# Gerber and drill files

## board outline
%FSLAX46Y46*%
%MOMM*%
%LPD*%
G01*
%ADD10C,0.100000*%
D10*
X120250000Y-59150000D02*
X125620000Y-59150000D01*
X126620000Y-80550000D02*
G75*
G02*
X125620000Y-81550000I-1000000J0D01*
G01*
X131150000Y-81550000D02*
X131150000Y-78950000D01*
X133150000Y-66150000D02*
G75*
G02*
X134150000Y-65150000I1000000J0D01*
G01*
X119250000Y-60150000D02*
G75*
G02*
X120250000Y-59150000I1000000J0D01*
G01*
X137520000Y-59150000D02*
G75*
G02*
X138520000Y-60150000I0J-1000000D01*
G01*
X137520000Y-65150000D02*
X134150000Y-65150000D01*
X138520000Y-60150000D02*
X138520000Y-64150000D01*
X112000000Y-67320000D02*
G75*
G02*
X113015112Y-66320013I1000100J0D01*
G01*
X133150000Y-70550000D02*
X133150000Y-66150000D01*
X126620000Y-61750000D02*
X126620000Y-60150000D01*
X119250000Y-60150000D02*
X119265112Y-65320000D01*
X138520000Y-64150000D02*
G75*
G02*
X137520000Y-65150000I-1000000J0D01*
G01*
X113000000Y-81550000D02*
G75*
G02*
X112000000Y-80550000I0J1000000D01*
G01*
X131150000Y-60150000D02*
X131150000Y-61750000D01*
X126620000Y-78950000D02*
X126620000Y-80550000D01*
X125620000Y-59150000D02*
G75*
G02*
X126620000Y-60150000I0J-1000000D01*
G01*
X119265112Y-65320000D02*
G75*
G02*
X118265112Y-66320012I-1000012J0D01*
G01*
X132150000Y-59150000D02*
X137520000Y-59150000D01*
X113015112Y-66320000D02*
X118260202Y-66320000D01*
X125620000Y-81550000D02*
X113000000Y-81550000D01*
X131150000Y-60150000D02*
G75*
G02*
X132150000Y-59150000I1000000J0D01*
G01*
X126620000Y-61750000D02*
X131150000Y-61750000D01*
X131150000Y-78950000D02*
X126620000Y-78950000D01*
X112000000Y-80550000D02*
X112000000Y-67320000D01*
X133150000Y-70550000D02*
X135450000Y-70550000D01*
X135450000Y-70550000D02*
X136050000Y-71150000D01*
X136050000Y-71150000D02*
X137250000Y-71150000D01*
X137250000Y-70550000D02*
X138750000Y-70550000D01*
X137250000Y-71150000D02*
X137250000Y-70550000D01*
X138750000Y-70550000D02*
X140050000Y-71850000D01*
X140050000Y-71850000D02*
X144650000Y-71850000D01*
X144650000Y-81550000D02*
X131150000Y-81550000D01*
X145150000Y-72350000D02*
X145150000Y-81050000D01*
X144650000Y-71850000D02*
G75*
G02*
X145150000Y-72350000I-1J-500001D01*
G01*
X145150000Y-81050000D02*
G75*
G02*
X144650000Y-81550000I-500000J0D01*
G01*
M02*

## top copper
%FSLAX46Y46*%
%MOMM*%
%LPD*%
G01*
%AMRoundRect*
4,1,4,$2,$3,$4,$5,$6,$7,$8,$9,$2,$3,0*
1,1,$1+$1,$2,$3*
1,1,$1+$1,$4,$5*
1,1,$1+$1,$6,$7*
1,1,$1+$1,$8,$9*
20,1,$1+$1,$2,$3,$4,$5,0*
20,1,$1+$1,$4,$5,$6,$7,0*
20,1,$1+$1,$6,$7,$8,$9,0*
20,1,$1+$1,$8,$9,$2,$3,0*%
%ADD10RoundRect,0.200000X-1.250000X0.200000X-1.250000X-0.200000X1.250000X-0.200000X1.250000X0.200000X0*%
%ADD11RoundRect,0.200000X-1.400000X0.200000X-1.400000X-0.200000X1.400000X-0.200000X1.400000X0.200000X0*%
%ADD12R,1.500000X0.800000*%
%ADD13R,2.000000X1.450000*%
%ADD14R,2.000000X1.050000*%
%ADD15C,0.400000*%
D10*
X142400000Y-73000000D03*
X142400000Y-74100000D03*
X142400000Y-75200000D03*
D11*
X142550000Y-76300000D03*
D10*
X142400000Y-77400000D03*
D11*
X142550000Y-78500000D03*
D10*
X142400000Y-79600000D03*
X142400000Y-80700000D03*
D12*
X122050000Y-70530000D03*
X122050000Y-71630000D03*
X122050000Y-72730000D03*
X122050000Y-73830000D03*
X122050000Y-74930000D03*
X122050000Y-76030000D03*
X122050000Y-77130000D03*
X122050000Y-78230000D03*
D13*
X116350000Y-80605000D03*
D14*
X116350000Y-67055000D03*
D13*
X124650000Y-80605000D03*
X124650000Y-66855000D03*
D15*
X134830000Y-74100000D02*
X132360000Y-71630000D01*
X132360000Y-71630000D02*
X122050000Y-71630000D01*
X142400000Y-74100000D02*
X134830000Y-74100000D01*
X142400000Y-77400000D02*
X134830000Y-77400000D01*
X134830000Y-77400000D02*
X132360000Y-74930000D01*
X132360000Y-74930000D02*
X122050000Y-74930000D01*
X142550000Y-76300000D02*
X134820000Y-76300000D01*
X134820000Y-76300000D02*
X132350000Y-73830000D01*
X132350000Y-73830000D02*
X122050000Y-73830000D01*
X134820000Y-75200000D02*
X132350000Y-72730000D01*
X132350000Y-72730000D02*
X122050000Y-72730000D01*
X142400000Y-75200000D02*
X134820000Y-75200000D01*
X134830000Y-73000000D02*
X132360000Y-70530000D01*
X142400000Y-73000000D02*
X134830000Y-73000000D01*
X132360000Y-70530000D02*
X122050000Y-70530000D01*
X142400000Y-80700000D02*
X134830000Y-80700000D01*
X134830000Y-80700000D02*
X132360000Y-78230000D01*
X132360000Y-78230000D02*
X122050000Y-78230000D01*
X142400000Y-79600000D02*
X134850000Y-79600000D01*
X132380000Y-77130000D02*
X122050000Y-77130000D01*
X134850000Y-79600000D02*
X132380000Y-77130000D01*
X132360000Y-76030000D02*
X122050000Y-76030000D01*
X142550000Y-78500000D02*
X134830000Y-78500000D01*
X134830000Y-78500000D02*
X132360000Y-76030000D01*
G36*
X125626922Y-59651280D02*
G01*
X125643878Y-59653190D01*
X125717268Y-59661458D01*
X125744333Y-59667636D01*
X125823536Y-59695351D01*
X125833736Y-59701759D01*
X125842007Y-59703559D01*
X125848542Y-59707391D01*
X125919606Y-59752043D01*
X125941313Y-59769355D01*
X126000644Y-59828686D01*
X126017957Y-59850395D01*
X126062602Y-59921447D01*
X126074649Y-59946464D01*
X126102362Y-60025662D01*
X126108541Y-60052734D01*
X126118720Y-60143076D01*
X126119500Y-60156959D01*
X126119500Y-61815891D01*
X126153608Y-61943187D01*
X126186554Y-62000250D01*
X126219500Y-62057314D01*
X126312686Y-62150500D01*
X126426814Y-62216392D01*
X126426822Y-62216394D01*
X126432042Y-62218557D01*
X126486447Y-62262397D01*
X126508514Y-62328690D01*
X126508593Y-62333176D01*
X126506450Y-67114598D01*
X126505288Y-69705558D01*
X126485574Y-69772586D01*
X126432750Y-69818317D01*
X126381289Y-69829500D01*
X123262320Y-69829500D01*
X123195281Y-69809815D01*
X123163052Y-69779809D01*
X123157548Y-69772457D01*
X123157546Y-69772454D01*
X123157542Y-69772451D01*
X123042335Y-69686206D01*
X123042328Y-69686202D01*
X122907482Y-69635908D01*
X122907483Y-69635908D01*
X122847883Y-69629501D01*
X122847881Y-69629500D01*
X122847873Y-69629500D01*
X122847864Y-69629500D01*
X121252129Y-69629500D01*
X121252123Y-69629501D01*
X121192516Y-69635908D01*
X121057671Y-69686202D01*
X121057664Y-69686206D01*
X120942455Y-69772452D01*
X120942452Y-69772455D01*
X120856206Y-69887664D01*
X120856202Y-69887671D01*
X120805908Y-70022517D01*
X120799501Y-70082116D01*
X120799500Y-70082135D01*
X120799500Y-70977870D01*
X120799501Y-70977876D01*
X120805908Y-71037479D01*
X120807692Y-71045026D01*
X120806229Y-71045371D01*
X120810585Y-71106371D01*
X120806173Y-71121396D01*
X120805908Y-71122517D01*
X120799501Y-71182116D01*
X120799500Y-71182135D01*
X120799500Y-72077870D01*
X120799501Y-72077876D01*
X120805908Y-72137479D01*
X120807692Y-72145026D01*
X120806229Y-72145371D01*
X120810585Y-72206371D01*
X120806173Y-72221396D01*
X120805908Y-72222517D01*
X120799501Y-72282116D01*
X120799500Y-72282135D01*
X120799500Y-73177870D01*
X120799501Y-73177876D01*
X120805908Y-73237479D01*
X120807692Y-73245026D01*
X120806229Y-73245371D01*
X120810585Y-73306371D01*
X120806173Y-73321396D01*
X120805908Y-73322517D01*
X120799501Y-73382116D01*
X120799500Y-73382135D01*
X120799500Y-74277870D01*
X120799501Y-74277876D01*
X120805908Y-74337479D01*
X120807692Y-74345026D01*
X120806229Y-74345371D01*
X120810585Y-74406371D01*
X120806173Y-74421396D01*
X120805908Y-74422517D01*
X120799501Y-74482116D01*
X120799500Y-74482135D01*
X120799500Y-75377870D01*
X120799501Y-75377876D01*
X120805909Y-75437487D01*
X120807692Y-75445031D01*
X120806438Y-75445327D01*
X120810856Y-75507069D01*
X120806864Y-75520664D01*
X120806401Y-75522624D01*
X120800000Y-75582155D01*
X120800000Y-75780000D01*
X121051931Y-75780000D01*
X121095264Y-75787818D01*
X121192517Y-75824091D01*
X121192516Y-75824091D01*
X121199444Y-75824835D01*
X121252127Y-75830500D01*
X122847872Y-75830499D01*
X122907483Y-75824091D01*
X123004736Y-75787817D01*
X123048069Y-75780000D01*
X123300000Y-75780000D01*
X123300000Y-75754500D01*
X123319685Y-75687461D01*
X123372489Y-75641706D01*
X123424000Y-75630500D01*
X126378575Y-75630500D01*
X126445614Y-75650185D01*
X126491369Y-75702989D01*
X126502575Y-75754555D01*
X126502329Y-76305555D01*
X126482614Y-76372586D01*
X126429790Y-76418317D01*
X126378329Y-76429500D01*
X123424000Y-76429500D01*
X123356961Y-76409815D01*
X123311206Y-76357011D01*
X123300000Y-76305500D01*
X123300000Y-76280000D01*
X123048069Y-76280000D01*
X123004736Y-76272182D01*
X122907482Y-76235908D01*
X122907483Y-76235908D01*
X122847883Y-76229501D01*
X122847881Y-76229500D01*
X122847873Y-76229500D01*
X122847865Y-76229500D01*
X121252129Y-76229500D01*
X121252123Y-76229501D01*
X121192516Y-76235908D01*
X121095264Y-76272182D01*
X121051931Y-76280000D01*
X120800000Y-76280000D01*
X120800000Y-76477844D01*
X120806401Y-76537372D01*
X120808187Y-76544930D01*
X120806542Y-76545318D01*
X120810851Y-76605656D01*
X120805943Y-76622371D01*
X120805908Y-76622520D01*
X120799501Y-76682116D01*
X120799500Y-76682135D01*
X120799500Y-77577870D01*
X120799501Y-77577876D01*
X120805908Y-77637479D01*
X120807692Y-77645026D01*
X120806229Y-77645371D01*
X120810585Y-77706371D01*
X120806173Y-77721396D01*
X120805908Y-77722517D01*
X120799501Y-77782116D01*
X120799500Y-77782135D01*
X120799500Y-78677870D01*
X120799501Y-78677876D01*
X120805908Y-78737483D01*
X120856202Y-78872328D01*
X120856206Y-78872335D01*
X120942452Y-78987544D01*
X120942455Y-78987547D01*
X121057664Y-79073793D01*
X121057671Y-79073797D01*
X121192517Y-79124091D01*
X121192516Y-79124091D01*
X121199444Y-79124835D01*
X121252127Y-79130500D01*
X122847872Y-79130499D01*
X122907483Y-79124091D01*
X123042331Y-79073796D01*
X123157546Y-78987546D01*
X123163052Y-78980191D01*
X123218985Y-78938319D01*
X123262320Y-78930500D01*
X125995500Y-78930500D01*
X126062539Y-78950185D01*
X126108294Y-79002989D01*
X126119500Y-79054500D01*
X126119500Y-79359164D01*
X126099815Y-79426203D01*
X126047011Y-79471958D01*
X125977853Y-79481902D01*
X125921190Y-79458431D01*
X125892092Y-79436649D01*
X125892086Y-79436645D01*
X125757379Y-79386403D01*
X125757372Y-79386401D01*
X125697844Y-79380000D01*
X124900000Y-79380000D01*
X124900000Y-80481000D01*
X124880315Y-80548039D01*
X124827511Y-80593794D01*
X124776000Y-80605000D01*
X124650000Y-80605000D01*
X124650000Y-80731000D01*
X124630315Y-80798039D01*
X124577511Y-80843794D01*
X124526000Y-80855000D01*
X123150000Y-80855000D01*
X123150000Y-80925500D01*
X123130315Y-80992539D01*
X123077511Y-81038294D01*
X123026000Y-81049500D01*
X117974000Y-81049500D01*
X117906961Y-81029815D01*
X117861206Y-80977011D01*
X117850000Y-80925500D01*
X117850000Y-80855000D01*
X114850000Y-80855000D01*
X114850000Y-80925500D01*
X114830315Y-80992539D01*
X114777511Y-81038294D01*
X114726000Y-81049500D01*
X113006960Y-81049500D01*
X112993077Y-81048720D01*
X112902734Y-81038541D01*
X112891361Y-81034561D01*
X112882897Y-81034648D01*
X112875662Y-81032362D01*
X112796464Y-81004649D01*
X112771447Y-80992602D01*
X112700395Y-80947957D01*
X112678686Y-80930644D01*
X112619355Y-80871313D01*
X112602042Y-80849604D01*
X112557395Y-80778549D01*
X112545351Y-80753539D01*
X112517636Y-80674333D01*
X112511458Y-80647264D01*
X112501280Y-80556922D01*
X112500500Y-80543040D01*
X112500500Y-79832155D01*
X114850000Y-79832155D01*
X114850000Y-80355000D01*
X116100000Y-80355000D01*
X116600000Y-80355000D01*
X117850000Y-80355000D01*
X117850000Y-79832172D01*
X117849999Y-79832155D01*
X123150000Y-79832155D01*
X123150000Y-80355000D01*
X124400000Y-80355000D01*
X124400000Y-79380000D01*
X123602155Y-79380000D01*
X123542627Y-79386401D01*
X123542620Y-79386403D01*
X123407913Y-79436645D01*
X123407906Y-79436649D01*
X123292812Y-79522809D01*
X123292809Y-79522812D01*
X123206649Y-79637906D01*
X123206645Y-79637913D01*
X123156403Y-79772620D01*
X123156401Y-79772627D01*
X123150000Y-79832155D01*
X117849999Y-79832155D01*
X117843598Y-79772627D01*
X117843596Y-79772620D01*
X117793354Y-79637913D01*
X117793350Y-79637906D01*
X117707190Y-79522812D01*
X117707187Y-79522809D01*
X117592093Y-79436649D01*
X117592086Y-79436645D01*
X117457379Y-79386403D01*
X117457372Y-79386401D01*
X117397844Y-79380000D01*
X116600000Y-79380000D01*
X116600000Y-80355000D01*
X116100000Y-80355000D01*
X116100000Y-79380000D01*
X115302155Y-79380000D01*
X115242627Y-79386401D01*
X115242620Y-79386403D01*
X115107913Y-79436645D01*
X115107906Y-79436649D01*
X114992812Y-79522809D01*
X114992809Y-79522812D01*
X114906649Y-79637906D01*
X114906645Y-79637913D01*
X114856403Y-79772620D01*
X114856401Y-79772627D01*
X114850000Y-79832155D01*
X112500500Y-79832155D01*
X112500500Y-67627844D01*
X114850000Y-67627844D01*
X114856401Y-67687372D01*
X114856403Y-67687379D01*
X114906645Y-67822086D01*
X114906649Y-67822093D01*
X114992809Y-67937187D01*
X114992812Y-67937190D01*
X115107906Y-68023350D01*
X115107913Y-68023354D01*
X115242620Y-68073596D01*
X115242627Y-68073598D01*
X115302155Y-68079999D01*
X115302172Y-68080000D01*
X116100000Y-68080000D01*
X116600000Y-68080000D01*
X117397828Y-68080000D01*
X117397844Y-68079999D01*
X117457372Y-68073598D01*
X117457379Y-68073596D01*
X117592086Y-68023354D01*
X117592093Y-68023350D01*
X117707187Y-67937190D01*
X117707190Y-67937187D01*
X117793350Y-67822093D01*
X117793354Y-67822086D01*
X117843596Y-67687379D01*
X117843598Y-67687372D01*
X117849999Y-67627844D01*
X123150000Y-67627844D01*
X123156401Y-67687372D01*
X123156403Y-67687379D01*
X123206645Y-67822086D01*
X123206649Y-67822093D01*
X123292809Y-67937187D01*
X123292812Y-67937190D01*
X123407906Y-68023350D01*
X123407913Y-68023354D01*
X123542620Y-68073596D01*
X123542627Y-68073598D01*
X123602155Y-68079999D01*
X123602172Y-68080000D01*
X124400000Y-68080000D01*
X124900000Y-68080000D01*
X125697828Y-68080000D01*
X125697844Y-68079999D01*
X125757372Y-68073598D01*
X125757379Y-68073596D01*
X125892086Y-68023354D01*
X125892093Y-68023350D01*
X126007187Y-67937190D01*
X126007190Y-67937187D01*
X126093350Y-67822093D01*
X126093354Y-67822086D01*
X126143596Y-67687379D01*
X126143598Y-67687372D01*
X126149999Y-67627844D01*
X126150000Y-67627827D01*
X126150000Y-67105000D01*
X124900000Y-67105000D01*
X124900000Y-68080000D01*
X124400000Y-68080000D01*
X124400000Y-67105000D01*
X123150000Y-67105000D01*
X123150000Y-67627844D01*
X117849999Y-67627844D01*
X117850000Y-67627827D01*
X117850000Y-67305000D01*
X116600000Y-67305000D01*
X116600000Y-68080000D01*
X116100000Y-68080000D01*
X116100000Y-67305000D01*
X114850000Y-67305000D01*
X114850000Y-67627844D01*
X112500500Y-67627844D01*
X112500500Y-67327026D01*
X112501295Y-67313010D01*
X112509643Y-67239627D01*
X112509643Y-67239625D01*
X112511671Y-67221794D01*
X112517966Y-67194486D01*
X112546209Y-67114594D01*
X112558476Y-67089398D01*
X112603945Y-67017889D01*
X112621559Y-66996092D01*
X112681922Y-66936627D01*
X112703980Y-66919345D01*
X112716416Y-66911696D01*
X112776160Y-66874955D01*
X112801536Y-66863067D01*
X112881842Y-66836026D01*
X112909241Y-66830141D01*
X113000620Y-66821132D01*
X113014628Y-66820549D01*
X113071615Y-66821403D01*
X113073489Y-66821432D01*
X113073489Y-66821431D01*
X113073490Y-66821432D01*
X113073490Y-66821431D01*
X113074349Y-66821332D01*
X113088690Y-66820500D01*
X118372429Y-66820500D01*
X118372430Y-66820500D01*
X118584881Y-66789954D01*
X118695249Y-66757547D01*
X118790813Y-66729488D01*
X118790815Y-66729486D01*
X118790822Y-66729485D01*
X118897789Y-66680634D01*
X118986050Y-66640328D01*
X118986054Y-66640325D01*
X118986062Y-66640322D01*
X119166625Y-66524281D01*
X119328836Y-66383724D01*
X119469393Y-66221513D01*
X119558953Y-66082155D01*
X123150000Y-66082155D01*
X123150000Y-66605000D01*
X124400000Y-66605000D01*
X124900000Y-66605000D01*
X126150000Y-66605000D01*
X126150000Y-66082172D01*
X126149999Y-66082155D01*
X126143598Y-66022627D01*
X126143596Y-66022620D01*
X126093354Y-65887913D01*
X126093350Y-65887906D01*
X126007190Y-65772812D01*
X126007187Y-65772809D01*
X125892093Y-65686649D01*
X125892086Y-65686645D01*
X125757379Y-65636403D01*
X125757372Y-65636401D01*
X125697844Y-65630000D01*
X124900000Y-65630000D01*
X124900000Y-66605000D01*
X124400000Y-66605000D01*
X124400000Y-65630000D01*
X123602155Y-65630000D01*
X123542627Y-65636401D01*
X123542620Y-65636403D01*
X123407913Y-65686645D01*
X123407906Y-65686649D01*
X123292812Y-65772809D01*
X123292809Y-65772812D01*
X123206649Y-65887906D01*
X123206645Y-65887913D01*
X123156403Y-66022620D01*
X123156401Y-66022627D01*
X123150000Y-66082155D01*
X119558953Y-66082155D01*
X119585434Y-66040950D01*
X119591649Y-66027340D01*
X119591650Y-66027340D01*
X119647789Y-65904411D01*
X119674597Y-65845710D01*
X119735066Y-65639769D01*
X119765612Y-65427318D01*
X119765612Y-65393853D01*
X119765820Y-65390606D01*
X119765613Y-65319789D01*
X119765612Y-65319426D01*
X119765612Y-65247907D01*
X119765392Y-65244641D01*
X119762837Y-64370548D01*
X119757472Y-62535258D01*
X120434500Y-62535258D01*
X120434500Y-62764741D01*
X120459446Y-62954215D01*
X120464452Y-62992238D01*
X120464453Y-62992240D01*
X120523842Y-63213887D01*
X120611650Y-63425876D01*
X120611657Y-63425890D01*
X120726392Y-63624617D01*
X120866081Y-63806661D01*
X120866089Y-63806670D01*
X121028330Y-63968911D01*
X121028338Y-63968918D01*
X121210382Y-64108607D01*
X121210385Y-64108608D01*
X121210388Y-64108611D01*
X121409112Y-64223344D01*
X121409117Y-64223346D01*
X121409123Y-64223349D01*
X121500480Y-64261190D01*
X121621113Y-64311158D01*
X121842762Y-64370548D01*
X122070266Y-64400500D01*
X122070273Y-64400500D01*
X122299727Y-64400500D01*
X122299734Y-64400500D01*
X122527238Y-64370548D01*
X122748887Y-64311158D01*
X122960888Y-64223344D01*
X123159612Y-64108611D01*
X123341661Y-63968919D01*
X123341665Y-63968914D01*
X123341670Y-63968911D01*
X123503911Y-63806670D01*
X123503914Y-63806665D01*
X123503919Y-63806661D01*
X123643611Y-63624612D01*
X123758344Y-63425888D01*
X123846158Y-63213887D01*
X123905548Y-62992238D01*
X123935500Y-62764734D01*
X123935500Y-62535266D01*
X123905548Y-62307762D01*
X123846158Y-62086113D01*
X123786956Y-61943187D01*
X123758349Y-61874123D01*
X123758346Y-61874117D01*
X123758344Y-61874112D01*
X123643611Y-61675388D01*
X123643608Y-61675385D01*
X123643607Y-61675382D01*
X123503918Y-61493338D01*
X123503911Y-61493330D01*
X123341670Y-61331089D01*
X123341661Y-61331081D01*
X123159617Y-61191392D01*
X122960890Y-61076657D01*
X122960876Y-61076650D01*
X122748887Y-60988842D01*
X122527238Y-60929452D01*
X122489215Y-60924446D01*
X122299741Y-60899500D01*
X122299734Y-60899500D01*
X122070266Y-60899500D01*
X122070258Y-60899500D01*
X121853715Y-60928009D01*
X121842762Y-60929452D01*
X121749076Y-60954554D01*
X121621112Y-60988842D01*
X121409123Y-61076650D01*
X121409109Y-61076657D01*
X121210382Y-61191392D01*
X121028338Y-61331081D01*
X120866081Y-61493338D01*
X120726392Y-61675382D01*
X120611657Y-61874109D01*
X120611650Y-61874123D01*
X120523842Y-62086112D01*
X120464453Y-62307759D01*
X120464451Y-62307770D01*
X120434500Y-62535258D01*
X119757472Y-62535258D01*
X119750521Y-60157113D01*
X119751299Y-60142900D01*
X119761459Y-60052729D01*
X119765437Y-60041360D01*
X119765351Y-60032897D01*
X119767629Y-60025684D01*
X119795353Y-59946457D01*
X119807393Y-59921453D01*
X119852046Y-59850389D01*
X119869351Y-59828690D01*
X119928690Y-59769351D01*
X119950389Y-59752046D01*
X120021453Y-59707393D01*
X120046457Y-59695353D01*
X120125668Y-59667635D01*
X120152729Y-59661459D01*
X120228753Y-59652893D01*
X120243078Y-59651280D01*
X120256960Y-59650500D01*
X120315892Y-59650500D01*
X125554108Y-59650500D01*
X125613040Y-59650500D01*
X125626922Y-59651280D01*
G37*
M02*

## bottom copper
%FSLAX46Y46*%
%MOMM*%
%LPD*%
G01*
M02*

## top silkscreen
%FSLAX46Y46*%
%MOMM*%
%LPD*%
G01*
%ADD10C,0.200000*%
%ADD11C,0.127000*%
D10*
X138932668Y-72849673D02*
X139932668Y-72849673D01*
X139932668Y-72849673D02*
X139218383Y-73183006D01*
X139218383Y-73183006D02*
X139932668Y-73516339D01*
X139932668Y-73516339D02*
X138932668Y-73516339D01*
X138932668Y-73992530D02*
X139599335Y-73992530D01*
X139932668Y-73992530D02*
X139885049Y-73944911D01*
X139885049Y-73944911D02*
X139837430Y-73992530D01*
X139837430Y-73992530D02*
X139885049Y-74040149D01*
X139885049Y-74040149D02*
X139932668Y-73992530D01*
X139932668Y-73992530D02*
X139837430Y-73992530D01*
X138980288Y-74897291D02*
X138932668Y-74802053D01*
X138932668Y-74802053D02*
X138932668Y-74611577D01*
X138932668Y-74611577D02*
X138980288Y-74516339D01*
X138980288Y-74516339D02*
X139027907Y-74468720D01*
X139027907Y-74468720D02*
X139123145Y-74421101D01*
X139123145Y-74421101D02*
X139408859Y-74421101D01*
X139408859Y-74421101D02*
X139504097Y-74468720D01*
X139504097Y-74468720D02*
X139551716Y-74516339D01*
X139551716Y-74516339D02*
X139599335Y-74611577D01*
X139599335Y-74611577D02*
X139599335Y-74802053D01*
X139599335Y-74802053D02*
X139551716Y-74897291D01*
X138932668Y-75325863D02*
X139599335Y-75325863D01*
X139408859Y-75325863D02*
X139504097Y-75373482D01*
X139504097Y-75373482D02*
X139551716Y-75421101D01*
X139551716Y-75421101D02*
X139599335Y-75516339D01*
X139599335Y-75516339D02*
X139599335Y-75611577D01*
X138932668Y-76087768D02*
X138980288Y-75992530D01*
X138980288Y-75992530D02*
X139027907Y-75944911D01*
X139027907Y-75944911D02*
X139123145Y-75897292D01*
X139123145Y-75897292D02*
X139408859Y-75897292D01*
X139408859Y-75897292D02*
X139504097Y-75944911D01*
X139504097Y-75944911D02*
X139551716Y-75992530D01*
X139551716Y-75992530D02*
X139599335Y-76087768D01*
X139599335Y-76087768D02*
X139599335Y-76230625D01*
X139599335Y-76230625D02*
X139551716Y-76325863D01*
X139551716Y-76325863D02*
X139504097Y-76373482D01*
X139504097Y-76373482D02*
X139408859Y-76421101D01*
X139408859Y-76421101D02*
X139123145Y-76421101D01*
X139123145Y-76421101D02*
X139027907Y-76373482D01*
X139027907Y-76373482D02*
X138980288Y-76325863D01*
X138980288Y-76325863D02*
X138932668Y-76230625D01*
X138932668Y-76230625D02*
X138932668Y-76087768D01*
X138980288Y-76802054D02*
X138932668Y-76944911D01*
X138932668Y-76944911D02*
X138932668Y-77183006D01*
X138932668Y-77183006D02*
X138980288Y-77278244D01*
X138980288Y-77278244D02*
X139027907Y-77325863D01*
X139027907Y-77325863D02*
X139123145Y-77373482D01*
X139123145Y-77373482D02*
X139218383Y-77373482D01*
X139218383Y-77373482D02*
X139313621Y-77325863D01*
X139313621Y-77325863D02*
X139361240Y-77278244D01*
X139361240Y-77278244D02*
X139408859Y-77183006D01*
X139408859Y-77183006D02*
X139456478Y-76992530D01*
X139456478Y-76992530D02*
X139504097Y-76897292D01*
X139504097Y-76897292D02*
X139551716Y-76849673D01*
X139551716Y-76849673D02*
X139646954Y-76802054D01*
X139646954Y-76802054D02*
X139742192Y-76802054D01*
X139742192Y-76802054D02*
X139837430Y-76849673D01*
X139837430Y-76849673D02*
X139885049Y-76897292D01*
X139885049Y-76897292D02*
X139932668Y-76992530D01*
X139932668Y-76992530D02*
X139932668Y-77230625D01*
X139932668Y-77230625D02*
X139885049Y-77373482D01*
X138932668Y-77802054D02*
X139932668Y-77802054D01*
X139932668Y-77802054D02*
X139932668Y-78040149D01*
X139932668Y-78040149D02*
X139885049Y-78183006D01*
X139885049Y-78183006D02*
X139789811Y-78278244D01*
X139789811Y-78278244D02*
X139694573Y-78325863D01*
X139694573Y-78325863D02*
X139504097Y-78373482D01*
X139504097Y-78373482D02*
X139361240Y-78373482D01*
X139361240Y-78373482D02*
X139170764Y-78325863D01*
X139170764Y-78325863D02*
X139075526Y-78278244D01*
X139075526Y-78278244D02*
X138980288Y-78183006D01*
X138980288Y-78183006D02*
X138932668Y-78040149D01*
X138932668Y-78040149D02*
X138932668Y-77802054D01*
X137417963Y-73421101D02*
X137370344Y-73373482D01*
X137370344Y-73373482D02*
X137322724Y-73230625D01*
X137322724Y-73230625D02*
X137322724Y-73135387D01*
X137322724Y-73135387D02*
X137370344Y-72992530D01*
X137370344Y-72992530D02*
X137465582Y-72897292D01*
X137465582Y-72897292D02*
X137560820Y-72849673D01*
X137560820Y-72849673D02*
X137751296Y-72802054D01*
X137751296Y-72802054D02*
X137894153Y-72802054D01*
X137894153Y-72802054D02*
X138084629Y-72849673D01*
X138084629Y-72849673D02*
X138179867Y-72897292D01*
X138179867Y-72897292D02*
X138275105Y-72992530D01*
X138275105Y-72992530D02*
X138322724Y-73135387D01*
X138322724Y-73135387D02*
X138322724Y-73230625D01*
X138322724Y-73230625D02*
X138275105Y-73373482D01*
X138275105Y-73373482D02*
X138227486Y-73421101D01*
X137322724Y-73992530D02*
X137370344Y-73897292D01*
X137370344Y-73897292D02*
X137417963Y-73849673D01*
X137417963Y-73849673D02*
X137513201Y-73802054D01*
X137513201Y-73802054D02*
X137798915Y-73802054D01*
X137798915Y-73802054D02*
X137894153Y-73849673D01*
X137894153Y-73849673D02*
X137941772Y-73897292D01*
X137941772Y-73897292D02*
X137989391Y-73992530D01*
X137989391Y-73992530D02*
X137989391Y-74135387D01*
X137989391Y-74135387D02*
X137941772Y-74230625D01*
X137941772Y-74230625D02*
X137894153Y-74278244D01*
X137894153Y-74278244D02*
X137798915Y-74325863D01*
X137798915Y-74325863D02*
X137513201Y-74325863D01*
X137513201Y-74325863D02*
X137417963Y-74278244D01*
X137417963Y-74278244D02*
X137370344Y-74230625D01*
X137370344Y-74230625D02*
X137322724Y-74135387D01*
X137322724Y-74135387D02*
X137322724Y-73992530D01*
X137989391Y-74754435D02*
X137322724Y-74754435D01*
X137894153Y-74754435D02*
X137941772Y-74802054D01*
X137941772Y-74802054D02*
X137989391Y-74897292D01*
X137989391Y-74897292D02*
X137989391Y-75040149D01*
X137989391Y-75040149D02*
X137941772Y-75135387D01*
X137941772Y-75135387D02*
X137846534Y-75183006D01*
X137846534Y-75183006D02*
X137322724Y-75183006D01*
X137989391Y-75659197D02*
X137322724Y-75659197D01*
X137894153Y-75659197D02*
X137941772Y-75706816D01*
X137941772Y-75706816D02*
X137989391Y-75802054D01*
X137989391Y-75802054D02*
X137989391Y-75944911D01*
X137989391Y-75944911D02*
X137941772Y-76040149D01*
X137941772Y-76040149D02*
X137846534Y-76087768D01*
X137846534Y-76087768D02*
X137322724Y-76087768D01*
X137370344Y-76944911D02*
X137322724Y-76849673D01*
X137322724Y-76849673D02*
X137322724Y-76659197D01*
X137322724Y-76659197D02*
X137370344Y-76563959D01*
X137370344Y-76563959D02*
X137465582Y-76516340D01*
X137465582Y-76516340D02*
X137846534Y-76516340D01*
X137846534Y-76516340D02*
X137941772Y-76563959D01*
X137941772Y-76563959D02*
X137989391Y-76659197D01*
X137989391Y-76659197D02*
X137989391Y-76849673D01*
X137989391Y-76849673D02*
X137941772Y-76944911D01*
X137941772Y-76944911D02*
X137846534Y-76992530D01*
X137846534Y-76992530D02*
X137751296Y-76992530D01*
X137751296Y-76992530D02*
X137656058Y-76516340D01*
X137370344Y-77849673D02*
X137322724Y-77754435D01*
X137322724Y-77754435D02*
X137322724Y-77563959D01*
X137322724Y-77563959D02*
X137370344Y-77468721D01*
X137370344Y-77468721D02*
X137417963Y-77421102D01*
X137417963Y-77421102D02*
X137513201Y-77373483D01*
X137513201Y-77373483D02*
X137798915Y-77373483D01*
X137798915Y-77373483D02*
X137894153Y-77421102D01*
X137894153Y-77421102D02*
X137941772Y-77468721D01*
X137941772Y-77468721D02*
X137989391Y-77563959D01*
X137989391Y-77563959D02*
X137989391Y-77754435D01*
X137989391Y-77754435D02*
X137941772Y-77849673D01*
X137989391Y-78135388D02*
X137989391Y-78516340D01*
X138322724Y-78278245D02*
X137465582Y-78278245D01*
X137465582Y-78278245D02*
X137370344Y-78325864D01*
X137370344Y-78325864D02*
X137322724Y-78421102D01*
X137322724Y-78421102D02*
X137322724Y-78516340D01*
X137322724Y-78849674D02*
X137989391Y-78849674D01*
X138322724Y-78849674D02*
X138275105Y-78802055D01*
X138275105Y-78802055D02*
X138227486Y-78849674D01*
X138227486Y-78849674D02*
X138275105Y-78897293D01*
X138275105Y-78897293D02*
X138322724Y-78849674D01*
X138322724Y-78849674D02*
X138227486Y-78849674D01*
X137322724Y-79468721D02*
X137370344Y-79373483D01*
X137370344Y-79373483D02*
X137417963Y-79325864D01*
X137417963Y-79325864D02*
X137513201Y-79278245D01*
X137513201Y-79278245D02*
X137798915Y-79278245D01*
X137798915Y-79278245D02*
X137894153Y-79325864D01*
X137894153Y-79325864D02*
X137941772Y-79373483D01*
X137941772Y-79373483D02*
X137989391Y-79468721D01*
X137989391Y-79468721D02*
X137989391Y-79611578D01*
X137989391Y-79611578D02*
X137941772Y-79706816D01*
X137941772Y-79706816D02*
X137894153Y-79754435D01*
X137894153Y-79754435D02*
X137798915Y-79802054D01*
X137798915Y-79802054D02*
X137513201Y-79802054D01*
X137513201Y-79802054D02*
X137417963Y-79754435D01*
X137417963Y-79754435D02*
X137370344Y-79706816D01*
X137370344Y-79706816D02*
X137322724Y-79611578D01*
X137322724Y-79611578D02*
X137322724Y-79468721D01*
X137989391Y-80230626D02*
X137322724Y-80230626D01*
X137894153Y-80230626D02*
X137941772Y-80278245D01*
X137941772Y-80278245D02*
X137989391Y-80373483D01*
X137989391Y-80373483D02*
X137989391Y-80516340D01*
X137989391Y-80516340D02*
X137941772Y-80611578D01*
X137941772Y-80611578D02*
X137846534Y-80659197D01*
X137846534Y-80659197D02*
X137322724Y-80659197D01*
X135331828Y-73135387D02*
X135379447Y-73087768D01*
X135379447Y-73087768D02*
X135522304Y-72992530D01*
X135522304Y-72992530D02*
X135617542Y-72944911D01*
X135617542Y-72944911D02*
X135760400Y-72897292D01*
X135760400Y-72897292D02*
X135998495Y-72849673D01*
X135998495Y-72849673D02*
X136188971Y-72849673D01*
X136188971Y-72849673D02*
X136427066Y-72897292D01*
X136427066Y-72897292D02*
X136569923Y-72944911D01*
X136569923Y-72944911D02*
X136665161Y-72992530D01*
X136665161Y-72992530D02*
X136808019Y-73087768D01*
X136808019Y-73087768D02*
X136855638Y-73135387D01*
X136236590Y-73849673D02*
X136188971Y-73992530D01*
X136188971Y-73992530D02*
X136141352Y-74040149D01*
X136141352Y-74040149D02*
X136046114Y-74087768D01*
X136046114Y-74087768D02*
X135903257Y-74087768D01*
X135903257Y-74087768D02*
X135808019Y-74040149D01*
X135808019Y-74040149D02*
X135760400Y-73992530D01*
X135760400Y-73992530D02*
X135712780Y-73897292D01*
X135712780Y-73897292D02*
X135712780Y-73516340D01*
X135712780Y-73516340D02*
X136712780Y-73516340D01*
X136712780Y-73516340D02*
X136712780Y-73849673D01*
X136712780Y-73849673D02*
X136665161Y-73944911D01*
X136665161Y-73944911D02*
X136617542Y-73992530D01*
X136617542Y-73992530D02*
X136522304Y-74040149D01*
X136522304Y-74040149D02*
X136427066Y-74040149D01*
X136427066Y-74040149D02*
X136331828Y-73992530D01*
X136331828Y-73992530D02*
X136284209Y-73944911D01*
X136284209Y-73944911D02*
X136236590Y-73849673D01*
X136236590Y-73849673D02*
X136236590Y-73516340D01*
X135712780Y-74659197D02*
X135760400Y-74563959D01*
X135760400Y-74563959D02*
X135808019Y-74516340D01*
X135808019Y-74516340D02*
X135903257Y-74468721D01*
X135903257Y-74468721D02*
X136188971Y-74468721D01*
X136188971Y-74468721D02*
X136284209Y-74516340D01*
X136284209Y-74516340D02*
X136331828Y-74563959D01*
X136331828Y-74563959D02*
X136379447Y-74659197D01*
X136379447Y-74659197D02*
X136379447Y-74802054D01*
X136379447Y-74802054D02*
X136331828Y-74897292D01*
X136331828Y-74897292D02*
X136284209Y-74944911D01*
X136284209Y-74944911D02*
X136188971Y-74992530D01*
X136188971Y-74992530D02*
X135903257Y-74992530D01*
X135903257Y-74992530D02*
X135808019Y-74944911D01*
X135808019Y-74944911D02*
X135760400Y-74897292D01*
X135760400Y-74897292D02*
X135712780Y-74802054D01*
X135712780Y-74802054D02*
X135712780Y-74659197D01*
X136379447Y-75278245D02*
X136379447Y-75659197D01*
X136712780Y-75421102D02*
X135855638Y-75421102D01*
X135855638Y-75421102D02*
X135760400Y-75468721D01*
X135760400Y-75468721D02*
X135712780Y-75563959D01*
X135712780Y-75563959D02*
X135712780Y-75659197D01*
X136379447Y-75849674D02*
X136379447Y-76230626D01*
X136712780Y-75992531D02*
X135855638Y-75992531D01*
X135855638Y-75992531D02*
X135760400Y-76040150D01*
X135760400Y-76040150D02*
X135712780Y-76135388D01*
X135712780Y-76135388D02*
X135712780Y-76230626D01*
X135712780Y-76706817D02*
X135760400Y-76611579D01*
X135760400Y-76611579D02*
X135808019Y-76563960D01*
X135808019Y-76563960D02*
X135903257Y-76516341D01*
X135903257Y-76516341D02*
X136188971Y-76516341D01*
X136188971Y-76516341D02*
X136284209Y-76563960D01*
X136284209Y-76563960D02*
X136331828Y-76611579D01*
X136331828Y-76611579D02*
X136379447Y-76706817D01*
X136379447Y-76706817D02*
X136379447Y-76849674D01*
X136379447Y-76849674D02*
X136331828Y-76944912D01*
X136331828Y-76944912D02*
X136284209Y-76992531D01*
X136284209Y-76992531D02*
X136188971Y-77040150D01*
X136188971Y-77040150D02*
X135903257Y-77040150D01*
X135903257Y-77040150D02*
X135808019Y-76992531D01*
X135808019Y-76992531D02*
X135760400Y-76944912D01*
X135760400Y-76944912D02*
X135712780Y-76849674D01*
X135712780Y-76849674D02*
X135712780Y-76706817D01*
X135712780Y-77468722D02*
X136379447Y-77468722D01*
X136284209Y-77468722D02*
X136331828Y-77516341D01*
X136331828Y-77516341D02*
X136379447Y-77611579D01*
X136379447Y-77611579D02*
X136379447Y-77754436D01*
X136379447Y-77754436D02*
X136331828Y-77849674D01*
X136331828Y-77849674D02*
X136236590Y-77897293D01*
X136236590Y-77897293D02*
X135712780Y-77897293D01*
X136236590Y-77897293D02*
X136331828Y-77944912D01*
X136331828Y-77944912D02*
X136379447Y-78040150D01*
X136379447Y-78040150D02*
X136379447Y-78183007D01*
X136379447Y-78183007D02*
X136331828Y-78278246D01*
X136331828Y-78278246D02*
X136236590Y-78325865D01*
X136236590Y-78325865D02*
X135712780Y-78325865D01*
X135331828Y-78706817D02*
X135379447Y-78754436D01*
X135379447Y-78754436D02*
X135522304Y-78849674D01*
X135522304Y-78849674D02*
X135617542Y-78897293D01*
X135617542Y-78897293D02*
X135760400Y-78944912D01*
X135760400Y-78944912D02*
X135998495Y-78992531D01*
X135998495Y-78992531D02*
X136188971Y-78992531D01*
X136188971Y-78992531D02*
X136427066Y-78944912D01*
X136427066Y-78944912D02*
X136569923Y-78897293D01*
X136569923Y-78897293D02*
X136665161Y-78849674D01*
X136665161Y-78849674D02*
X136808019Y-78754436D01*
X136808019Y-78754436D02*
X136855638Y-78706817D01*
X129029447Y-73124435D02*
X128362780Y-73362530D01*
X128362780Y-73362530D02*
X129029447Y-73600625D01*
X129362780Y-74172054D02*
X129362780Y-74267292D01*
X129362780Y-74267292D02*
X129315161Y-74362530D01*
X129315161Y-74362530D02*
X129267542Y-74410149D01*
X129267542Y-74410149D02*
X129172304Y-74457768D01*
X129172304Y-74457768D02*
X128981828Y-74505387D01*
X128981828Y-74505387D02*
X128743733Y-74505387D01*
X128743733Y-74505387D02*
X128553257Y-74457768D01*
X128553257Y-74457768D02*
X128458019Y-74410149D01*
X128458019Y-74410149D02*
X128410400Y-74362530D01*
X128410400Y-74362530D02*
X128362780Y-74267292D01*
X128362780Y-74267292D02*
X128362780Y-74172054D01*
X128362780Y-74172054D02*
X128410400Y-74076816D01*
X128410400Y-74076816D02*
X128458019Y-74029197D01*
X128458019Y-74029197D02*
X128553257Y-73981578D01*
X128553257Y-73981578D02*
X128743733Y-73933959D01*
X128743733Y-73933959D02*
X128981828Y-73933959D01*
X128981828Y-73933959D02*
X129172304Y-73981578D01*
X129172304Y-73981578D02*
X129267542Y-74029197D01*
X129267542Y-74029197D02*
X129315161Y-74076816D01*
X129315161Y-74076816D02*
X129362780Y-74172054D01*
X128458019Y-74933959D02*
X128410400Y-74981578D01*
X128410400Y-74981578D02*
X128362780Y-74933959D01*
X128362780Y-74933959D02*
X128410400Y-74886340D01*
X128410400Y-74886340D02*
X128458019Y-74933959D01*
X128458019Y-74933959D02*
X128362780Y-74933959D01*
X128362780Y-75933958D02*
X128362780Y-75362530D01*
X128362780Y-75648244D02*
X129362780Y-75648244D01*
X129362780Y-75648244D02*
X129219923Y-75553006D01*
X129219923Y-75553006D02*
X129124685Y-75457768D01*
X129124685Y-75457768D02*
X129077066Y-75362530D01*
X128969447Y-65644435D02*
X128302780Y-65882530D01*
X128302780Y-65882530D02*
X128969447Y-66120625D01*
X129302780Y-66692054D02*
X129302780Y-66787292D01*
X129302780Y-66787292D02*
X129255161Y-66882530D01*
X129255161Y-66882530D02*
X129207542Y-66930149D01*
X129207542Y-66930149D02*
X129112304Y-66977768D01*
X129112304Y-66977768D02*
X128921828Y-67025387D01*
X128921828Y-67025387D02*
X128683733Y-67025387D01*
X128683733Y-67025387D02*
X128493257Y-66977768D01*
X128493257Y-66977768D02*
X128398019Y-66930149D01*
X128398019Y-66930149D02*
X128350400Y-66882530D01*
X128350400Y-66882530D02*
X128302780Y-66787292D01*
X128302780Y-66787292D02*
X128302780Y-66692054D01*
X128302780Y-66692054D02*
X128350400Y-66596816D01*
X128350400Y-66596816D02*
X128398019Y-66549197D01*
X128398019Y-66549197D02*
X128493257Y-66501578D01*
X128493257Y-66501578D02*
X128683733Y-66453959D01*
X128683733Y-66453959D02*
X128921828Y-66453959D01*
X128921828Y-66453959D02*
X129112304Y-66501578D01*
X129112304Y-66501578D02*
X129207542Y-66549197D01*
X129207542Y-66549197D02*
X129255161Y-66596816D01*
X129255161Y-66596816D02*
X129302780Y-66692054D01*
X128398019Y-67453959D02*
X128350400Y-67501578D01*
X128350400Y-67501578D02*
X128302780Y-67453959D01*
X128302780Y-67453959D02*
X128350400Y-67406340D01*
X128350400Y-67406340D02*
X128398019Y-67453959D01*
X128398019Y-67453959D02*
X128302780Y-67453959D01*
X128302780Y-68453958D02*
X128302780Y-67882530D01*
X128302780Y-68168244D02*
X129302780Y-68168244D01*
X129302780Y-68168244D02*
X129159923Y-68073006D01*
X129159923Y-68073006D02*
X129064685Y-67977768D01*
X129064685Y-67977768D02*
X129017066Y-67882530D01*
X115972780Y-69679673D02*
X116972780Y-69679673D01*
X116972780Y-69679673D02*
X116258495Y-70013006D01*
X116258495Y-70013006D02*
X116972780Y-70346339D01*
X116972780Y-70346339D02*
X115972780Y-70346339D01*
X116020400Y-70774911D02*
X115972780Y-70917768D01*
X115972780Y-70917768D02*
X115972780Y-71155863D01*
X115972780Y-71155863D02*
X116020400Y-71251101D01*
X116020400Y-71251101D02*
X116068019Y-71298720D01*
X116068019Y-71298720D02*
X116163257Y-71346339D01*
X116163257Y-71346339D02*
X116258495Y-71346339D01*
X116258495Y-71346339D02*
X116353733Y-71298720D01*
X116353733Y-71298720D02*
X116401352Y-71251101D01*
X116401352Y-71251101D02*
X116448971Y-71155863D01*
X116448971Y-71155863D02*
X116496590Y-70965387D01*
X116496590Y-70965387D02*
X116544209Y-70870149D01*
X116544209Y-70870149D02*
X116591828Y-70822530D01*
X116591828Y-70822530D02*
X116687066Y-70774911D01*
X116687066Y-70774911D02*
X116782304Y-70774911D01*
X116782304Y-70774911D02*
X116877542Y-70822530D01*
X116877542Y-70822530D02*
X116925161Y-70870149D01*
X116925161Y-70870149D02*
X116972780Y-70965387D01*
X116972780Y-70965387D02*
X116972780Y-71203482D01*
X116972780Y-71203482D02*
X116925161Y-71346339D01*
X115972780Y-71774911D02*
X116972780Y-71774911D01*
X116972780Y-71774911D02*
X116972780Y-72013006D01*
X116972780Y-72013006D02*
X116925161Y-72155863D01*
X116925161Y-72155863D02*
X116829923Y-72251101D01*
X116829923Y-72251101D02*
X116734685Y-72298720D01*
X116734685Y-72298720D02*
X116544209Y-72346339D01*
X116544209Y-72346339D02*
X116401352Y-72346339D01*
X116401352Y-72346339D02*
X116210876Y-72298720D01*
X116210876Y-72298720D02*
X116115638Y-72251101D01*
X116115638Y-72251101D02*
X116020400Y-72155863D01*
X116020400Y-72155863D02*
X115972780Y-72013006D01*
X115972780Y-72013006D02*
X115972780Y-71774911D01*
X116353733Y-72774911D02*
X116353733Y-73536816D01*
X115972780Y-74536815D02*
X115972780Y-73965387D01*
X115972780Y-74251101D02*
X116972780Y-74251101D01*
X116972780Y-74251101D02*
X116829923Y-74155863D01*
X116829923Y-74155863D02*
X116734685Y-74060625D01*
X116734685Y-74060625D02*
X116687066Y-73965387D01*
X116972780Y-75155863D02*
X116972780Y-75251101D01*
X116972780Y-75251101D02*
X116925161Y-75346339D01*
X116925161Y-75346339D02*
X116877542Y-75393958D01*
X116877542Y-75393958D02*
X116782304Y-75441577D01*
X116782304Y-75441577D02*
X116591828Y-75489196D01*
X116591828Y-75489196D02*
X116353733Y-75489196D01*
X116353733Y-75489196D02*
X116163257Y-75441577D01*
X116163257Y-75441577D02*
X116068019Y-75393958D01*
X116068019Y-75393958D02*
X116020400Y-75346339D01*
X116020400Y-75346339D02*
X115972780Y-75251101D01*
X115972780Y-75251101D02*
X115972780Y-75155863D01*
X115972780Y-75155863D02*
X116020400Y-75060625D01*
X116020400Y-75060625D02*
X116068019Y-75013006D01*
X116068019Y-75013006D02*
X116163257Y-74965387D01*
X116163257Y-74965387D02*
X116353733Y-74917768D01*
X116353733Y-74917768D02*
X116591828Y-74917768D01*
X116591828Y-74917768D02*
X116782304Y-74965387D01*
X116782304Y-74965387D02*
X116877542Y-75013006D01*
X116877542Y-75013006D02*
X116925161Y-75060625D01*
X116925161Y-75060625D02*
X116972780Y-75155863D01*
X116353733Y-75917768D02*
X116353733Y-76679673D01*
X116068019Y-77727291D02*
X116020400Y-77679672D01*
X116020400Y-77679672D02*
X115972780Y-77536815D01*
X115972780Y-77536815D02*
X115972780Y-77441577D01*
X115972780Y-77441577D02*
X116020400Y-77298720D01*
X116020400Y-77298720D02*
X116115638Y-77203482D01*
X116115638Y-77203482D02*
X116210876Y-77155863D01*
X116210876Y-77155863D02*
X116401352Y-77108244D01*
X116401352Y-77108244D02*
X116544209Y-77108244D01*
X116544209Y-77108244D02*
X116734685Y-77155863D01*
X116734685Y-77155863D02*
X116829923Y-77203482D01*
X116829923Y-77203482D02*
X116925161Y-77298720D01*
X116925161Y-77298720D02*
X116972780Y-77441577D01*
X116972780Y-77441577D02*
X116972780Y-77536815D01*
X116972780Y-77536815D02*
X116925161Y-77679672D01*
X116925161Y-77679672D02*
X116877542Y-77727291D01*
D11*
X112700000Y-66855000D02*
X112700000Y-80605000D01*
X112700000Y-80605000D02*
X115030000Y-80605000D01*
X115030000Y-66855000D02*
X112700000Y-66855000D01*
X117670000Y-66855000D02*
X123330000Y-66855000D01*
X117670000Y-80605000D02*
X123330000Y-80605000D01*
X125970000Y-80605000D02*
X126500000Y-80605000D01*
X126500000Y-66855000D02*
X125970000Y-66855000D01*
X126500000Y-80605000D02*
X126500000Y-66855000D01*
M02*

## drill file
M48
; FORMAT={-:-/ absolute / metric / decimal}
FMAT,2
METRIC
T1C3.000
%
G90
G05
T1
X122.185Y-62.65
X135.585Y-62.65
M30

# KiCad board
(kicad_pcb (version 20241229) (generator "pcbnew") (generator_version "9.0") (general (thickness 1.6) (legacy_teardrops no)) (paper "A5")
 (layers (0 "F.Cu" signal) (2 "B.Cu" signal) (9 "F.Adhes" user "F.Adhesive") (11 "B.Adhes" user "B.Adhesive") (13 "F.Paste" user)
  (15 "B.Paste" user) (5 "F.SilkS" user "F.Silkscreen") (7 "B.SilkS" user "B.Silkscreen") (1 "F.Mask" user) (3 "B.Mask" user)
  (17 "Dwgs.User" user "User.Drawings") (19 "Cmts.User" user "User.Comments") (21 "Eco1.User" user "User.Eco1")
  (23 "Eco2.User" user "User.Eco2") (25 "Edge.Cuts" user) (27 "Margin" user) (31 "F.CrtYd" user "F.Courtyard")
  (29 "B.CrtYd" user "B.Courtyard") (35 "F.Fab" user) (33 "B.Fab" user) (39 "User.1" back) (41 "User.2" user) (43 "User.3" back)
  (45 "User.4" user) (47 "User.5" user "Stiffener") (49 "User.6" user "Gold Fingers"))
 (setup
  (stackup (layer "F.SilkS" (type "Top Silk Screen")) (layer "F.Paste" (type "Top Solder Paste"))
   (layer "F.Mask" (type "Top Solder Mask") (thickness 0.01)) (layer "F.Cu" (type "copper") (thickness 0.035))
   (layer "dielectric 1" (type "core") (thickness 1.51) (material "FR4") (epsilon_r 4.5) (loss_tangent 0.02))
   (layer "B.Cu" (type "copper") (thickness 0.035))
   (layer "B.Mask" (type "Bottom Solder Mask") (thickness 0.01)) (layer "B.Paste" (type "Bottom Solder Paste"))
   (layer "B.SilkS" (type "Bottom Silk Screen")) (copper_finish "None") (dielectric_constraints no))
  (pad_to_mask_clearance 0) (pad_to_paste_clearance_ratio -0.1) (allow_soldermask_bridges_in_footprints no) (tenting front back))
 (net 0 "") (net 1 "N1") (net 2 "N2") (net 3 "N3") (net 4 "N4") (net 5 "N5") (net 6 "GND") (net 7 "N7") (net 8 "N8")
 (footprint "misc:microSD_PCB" (layer "F.Cu") (at 142.55 76.85 -90)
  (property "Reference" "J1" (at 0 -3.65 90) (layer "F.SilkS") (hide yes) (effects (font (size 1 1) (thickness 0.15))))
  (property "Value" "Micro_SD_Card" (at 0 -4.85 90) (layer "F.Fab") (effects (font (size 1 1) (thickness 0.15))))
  (fp_line (start -6.3 9.4) (end -6.3 7.1) (stroke (width 0.1) (type solid)) (layer "Edge.Cuts"))
  (fp_line (start -6.3 7.1) (end -5.7 6.5) (stroke (width 0.1) (type default)) (layer "Edge.Cuts"))
  (fp_line (start -5.7 6.5) (end -5.7 5.3) (stroke (width 0.1) (type default)) (layer "Edge.Cuts"))
  (fp_line (start -6.3 5.3) (end -6.3 3.8) (stroke (width 0.1) (type default)) (layer "Edge.Cuts"))
  (fp_line (start -5.7 5.3) (end -6.3 5.3) (stroke (width 0.1) (type default)) (layer "Edge.Cuts"))
  (fp_line (start -6.3 3.8) (end -5 2.5) (stroke (width 0.1) (type default)) (layer "Edge.Cuts"))
  (fp_line (start -5 2.5) (end -5 -2.1) (stroke (width 0.1) (type default)) (layer "Edge.Cuts"))
  (fp_line (start 4.7 -2.1) (end 4.7 11.4) (stroke (width 0.1) (type solid)) (layer "Edge.Cuts"))
  (fp_line (start -4.5 -2.6) (end 4.2 -2.6) (stroke (width 0.1) (type default)) (layer "Edge.Cuts"))
  (fp_arc (start -5 -2.1) (mid -4.853553 -2.453553) (end -4.5 -2.6) (stroke (width 0.1) (type default)) (layer "Edge.Cuts"))
  (fp_arc (start 4.2 -2.6) (mid 4.553553 -2.453553) (end 4.7 -2.1) (stroke (width 0.1) (type default)) (layer "Edge.Cuts"))
  (pad "1" smd roundrect (at -3.85 0.15 270) (size 0.8 2.9) (layers "F.Cu" "F.Mask") (roundrect_rratio 0.25) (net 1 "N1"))
  (pad "2" smd roundrect (at -2.75 0.15 270) (size 0.8 2.9) (layers "F.Cu" "F.Mask") (roundrect_rratio 0.25) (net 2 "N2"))
  (pad "3" smd roundrect (at -1.65 0.15 270) (size 0.8 2.9) (layers "F.Cu" "F.Mask") (roundrect_rratio 0.25) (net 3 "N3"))
  (pad "4" smd roundrect (at -0.55 0 270) (size 0.8 3.2) (layers "F.Cu" "F.Mask") (roundrect_rratio 0.25) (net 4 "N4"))
  (pad "5" smd roundrect (at 0.55 0.15 270) (size 0.8 2.9) (layers "F.Cu" "F.Mask") (roundrect_rratio 0.25) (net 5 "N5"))
  (pad "6" smd roundrect (at 1.65 0 270) (size 0.8 3.2) (layers "F.Cu" "F.Mask") (roundrect_rratio 0.25) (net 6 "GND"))
  (pad "7" smd roundrect (at 2.75 0.15 270) (size 0.8 2.9) (layers "F.Cu" "F.Mask") (roundrect_rratio 0.25) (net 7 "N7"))
  (pad "8" smd roundrect (at 3.85 0.15 270) (size 0.8 2.9) (layers "F.Cu" "F.Mask") (roundrect_rratio 0.25) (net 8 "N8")))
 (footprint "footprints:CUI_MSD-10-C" (layer "F.Cu") (at 119.6 73.73 90)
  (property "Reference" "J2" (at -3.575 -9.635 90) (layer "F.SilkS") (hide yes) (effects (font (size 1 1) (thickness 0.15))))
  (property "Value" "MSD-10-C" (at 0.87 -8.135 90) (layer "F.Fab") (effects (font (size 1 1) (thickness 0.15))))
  (fp_line (start 6.875 -6.9) (end -6.875 -6.9) (stroke (width 0.127) (type solid)) (layer "F.SilkS"))
  (fp_line (start -6.875 -6.9) (end -6.875 -4.57) (stroke (width 0.127) (type solid)) (layer "F.SilkS"))
  (fp_line (start 6.875 -4.57) (end 6.875 -6.9) (stroke (width 0.127) (type solid)) (layer "F.SilkS"))
  (fp_line (start 6.875 -1.93) (end 6.875 3.73) (stroke (width 0.127) (type solid)) (layer "F.SilkS"))
  (fp_line (start -6.875 -1.93) (end -6.875 3.73) (stroke (width 0.127) (type solid)) (layer "F.SilkS"))
  (fp_line (start -6.875 6.37) (end -6.875 6.9) (stroke (width 0.127) (type solid)) (layer "F.SilkS"))
  (fp_line (start 6.875 6.9) (end 6.875 6.37) (stroke (width 0.127) (type solid)) (layer "F.SilkS"))
  (fp_line (start -6.875 6.9) (end 6.875 6.9) (stroke (width 0.127) (type solid)) (layer "F.SilkS"))
  (pad "01" smd rect (at 3.2 2.45 90) (size 0.8 1.5) (layers "F.Cu" "F.Mask" "F.Paste") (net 1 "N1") (solder_mask_margin 0.102))
  (pad "02" smd rect (at 2.1 2.45 90) (size 0.8 1.5) (layers "F.Cu" "F.Mask" "F.Paste") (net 2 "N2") (solder_mask_margin 0.102))
  (pad "03" smd rect (at 1 2.45 90) (size 0.8 1.5) (layers "F.Cu" "F.Mask" "F.Paste") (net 3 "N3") (solder_mask_margin 0.102))
  (pad "04" smd rect (at -0.1 2.45 90) (size 0.8 1.5) (layers "F.Cu" "F.Mask" "F.Paste") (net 4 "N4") (solder_mask_margin 0.102))
  (pad "05" smd rect (at -1.2 2.45 90) (size 0.8 1.5) (layers "F.Cu" "F.Mask" "F.Paste") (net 5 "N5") (solder_mask_margin 0.102))
  (pad "06" smd rect (at -2.3 2.45 90) (size 0.8 1.5) (layers "F.Cu" "F.Mask" "F.Paste") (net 6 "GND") (solder_mask_margin 0.102))
  (pad "07" smd rect (at -3.4 2.45 90) (size 0.8 1.5) (layers "F.Cu" "F.Mask" "F.Paste") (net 7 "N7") (solder_mask_margin 0.102))
  (pad "08" smd rect (at -4.5 2.45 90) (size 0.8 1.5) (layers "F.Cu" "F.Mask" "F.Paste") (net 8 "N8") (solder_mask_margin 0.102))
  (pad "G1" smd rect (at -6.875 -3.25 90) (size 1.45 2) (layers "F.Cu" "F.Mask" "F.Paste") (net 6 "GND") (solder_mask_margin 0.102))
  (pad "G2" smd rect (at 6.675 -3.25 90) (size 1.05 2) (layers "F.Cu" "F.Mask" "F.Paste") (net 6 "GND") (solder_mask_margin 0.102))
  (pad "G3" smd rect (at -6.875 5.05 90) (size 1.45 2) (layers "F.Cu" "F.Mask" "F.Paste") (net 6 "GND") (solder_mask_margin 0.102))
  (pad "G4" smd rect (at 6.875 5.05 90) (size 1.45 2) (layers "F.Cu" "F.Mask" "F.Paste") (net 6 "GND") (solder_mask_margin 0.102)))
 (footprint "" (layer "F.Cu") (at 122.185 62.65)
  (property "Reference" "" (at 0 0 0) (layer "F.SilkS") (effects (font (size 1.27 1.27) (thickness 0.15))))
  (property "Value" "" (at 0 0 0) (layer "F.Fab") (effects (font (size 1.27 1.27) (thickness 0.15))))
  (pad "" np_thru_hole circle (at 0 0) (size 3 3) (drill 3) (layers "*.Cu" "*.Mask" "F.Paste") (solder_paste_margin_ratio 0)))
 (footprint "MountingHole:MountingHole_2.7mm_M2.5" (layer "F.Cu") (at 135.585 62.65)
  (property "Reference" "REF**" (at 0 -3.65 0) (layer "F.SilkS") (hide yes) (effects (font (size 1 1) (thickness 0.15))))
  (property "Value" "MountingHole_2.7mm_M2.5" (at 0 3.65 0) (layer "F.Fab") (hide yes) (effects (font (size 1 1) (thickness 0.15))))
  (pad "" np_thru_hole circle (at 0 0) (size 3 3) (drill 3) (layers "*.Cu" "*.Mask" "F.Paste") (solder_paste_margin_ratio 0)))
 (gr_line (start 120.25 59.15) (end 125.62 59.15) (stroke (width 0.1) (type solid)) (layer "Edge.Cuts"))
 (gr_arc (start 126.62 80.55) (mid 126.327107 81.257107) (end 125.62 81.55) (stroke (width 0.1) (type default)) (layer "Edge.Cuts"))
 (gr_line (start 131.15 81.55) (end 131.15 78.95) (stroke (width 0.1) (type solid)) (layer "Edge.Cuts"))
 (gr_arc (start 133.15 66.15) (mid 133.442893 65.442893) (end 134.15 65.15) (stroke (width 0.1) (type default)) (layer "Edge.Cuts"))
 (gr_arc (start 119.25 60.15) (mid 119.542893 59.442893) (end 120.25 59.15) (stroke (width 0.1) (type default)) (layer "Edge.Cuts"))
 (gr_arc (start 137.52 59.15) (mid 138.227107 59.442893) (end 138.52 60.15) (stroke (width 0.1) (type default)) (layer "Edge.Cuts"))
 (gr_line (start 137.52 65.15) (end 134.15 65.15) (stroke (width 0.1) (type solid)) (layer "Edge.Cuts"))
 (gr_line (start 138.52 60.15) (end 138.52 64.15) (stroke (width 0.1) (type solid)) (layer "Edge.Cuts"))
 (gr_arc (start 112 67.32) (mid 112.298249 66.60753) (end 113.015112 66.32) (stroke (width 0.1) (type solid)) (layer "Edge.Cuts"))
 (gr_line (start 133.15 70.55) (end 133.15 66.15) (stroke (width 0.1) (type solid)) (layer "Edge.Cuts"))
 (gr_line (start 126.62 61.75) (end 126.62 60.15) (stroke (width 0.1) (type solid)) (layer "Edge.Cuts"))
 (gr_line (start 119.25 60.15) (end 119.265112 65.32) (stroke (width 0.1) (type solid)) (layer "Edge.Cuts"))
 (gr_arc (start 138.52 64.15) (mid 138.227107 64.857107) (end 137.52 65.15) (stroke (width 0.1) (type default)) (layer "Edge.Cuts"))
 (gr_arc (start 113 81.55) (mid 112.292893 81.257107) (end 112 80.55) (stroke (width 0.1) (type default)) (layer "Edge.Cuts"))
 (gr_line (start 131.15 60.15) (end 131.15 61.75) (stroke (width 0.1) (type solid)) (layer "Edge.Cuts"))
 (gr_line (start 126.62 78.95) (end 126.62 80.55) (stroke (width 0.1) (type solid)) (layer "Edge.Cuts"))
 (gr_arc (start 125.62 59.15) (mid 126.327107 59.442893) (end 126.62 60.15) (stroke (width 0.1) (type default)) (layer "Edge.Cuts"))
 (gr_arc (start 119.265112 65.32) (mid 118.972219 66.027107) (end 118.265112 66.32) (stroke (width 0.1) (type default)) (layer "Edge.Cuts"))
 (gr_line (start 132.15 59.15) (end 137.52 59.15) (stroke (width 0.1) (type solid)) (layer "Edge.Cuts"))
 (gr_line (start 113.015112 66.32) (end 118.260202 66.32) (stroke (width 0.1) (type solid)) (layer "Edge.Cuts"))
 (gr_line (start 125.62 81.55) (end 113 81.55) (stroke (width 0.1) (type solid)) (layer "Edge.Cuts"))
 (gr_arc (start 131.15 60.15) (mid 131.442893 59.442893) (end 132.15 59.15) (stroke (width 0.1) (type default)) (layer "Edge.Cuts"))
 (gr_line (start 126.62 61.75) (end 131.15 61.75) (stroke (width 0.1) (type solid)) (layer "Edge.Cuts"))
 (gr_line (start 131.15 78.95) (end 126.62 78.95) (stroke (width 0.1) (type solid)) (layer "Edge.Cuts"))
 (gr_line (start 112 80.55) (end 112 67.32) (stroke (width 0.1) (type solid)) (layer "Edge.Cuts"))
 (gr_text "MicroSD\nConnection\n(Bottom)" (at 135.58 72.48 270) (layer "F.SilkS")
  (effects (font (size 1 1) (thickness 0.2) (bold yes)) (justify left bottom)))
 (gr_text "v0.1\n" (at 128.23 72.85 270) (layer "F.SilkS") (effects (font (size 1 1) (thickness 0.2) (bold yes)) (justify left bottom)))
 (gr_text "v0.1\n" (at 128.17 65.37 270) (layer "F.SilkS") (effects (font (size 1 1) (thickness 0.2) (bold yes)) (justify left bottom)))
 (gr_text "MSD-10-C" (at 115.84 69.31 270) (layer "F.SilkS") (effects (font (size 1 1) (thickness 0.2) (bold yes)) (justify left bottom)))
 (segment (start 134.83 74.1) (end 132.36 71.63) (width 0.4) (layer "F.Cu") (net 2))
 (segment (start 132.36 71.63) (end 122.05 71.63) (width 0.4) (layer "F.Cu") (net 2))
 (segment (start 142.4 74.1) (end 134.83 74.1) (width 0.4) (layer "F.Cu") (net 2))
 (segment (start 142.4 77.4) (end 134.83 77.4) (width 0.4) (layer "F.Cu") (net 5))
 (segment (start 134.83 77.4) (end 132.36 74.93) (width 0.4) (layer "F.Cu") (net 5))
 (segment (start 132.36 74.93) (end 122.05 74.93) (width 0.4) (layer "F.Cu") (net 5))
 (segment (start 142.55 76.3) (end 134.82 76.3) (width 0.4) (layer "F.Cu") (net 4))
 (segment (start 134.82 76.3) (end 132.35 73.83) (width 0.4) (layer "F.Cu") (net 4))
 (segment (start 132.35 73.83) (end 122.05 73.83) (width 0.4) (layer "F.Cu") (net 4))
 (segment (start 134.82 75.2) (end 132.35 72.73) (width 0.4) (layer "F.Cu") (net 3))
 (segment (start 132.35 72.73) (end 122.05 72.73) (width 0.4) (layer "F.Cu") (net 3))
 (segment (start 142.4 75.2) (end 134.82 75.2) (width 0.4) (layer "F.Cu") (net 3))
 (segment (start 134.83 73) (end 132.36 70.53) (width 0.4) (layer "F.Cu") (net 1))
 (segment (start 142.4 73) (end 134.83 73) (width 0.4) (layer "F.Cu") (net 1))
 (segment (start 132.36 70.53) (end 122.05 70.53) (width 0.4) (layer "F.Cu") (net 1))
 (segment (start 142.4 80.7) (end 134.83 80.7) (width 0.4) (layer "F.Cu") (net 8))
 (segment (start 134.83 80.7) (end 132.36 78.23) (width 0.4) (layer "F.Cu") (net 8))
 (segment (start 132.36 78.23) (end 122.05 78.23) (width 0.4) (layer "F.Cu") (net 8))
 (segment (start 142.4 79.6) (end 134.85 79.6) (width 0.4) (layer "F.Cu") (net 7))
 (segment (start 132.38 77.13) (end 122.05 77.13) (width 0.4) (layer "F.Cu") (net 7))
 (segment (start 134.85 79.6) (end 132.38 77.13) (width 0.4) (layer "F.Cu") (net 7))
 (segment (start 132.36 76.03) (end 122.05 76.03) (width 0.4) (layer "F.Cu") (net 6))
 (segment (start 142.55 78.5) (end 134.83 78.5) (width 0.4) (layer "F.Cu") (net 6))
 (segment (start 134.83 78.5) (end 132.36 76.03) (width 0.4) (layer "F.Cu") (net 6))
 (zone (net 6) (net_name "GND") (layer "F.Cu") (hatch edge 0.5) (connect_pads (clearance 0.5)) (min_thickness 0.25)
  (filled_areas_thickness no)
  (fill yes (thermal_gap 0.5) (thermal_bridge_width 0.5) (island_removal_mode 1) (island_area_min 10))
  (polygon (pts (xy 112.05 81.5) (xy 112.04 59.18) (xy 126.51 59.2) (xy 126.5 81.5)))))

